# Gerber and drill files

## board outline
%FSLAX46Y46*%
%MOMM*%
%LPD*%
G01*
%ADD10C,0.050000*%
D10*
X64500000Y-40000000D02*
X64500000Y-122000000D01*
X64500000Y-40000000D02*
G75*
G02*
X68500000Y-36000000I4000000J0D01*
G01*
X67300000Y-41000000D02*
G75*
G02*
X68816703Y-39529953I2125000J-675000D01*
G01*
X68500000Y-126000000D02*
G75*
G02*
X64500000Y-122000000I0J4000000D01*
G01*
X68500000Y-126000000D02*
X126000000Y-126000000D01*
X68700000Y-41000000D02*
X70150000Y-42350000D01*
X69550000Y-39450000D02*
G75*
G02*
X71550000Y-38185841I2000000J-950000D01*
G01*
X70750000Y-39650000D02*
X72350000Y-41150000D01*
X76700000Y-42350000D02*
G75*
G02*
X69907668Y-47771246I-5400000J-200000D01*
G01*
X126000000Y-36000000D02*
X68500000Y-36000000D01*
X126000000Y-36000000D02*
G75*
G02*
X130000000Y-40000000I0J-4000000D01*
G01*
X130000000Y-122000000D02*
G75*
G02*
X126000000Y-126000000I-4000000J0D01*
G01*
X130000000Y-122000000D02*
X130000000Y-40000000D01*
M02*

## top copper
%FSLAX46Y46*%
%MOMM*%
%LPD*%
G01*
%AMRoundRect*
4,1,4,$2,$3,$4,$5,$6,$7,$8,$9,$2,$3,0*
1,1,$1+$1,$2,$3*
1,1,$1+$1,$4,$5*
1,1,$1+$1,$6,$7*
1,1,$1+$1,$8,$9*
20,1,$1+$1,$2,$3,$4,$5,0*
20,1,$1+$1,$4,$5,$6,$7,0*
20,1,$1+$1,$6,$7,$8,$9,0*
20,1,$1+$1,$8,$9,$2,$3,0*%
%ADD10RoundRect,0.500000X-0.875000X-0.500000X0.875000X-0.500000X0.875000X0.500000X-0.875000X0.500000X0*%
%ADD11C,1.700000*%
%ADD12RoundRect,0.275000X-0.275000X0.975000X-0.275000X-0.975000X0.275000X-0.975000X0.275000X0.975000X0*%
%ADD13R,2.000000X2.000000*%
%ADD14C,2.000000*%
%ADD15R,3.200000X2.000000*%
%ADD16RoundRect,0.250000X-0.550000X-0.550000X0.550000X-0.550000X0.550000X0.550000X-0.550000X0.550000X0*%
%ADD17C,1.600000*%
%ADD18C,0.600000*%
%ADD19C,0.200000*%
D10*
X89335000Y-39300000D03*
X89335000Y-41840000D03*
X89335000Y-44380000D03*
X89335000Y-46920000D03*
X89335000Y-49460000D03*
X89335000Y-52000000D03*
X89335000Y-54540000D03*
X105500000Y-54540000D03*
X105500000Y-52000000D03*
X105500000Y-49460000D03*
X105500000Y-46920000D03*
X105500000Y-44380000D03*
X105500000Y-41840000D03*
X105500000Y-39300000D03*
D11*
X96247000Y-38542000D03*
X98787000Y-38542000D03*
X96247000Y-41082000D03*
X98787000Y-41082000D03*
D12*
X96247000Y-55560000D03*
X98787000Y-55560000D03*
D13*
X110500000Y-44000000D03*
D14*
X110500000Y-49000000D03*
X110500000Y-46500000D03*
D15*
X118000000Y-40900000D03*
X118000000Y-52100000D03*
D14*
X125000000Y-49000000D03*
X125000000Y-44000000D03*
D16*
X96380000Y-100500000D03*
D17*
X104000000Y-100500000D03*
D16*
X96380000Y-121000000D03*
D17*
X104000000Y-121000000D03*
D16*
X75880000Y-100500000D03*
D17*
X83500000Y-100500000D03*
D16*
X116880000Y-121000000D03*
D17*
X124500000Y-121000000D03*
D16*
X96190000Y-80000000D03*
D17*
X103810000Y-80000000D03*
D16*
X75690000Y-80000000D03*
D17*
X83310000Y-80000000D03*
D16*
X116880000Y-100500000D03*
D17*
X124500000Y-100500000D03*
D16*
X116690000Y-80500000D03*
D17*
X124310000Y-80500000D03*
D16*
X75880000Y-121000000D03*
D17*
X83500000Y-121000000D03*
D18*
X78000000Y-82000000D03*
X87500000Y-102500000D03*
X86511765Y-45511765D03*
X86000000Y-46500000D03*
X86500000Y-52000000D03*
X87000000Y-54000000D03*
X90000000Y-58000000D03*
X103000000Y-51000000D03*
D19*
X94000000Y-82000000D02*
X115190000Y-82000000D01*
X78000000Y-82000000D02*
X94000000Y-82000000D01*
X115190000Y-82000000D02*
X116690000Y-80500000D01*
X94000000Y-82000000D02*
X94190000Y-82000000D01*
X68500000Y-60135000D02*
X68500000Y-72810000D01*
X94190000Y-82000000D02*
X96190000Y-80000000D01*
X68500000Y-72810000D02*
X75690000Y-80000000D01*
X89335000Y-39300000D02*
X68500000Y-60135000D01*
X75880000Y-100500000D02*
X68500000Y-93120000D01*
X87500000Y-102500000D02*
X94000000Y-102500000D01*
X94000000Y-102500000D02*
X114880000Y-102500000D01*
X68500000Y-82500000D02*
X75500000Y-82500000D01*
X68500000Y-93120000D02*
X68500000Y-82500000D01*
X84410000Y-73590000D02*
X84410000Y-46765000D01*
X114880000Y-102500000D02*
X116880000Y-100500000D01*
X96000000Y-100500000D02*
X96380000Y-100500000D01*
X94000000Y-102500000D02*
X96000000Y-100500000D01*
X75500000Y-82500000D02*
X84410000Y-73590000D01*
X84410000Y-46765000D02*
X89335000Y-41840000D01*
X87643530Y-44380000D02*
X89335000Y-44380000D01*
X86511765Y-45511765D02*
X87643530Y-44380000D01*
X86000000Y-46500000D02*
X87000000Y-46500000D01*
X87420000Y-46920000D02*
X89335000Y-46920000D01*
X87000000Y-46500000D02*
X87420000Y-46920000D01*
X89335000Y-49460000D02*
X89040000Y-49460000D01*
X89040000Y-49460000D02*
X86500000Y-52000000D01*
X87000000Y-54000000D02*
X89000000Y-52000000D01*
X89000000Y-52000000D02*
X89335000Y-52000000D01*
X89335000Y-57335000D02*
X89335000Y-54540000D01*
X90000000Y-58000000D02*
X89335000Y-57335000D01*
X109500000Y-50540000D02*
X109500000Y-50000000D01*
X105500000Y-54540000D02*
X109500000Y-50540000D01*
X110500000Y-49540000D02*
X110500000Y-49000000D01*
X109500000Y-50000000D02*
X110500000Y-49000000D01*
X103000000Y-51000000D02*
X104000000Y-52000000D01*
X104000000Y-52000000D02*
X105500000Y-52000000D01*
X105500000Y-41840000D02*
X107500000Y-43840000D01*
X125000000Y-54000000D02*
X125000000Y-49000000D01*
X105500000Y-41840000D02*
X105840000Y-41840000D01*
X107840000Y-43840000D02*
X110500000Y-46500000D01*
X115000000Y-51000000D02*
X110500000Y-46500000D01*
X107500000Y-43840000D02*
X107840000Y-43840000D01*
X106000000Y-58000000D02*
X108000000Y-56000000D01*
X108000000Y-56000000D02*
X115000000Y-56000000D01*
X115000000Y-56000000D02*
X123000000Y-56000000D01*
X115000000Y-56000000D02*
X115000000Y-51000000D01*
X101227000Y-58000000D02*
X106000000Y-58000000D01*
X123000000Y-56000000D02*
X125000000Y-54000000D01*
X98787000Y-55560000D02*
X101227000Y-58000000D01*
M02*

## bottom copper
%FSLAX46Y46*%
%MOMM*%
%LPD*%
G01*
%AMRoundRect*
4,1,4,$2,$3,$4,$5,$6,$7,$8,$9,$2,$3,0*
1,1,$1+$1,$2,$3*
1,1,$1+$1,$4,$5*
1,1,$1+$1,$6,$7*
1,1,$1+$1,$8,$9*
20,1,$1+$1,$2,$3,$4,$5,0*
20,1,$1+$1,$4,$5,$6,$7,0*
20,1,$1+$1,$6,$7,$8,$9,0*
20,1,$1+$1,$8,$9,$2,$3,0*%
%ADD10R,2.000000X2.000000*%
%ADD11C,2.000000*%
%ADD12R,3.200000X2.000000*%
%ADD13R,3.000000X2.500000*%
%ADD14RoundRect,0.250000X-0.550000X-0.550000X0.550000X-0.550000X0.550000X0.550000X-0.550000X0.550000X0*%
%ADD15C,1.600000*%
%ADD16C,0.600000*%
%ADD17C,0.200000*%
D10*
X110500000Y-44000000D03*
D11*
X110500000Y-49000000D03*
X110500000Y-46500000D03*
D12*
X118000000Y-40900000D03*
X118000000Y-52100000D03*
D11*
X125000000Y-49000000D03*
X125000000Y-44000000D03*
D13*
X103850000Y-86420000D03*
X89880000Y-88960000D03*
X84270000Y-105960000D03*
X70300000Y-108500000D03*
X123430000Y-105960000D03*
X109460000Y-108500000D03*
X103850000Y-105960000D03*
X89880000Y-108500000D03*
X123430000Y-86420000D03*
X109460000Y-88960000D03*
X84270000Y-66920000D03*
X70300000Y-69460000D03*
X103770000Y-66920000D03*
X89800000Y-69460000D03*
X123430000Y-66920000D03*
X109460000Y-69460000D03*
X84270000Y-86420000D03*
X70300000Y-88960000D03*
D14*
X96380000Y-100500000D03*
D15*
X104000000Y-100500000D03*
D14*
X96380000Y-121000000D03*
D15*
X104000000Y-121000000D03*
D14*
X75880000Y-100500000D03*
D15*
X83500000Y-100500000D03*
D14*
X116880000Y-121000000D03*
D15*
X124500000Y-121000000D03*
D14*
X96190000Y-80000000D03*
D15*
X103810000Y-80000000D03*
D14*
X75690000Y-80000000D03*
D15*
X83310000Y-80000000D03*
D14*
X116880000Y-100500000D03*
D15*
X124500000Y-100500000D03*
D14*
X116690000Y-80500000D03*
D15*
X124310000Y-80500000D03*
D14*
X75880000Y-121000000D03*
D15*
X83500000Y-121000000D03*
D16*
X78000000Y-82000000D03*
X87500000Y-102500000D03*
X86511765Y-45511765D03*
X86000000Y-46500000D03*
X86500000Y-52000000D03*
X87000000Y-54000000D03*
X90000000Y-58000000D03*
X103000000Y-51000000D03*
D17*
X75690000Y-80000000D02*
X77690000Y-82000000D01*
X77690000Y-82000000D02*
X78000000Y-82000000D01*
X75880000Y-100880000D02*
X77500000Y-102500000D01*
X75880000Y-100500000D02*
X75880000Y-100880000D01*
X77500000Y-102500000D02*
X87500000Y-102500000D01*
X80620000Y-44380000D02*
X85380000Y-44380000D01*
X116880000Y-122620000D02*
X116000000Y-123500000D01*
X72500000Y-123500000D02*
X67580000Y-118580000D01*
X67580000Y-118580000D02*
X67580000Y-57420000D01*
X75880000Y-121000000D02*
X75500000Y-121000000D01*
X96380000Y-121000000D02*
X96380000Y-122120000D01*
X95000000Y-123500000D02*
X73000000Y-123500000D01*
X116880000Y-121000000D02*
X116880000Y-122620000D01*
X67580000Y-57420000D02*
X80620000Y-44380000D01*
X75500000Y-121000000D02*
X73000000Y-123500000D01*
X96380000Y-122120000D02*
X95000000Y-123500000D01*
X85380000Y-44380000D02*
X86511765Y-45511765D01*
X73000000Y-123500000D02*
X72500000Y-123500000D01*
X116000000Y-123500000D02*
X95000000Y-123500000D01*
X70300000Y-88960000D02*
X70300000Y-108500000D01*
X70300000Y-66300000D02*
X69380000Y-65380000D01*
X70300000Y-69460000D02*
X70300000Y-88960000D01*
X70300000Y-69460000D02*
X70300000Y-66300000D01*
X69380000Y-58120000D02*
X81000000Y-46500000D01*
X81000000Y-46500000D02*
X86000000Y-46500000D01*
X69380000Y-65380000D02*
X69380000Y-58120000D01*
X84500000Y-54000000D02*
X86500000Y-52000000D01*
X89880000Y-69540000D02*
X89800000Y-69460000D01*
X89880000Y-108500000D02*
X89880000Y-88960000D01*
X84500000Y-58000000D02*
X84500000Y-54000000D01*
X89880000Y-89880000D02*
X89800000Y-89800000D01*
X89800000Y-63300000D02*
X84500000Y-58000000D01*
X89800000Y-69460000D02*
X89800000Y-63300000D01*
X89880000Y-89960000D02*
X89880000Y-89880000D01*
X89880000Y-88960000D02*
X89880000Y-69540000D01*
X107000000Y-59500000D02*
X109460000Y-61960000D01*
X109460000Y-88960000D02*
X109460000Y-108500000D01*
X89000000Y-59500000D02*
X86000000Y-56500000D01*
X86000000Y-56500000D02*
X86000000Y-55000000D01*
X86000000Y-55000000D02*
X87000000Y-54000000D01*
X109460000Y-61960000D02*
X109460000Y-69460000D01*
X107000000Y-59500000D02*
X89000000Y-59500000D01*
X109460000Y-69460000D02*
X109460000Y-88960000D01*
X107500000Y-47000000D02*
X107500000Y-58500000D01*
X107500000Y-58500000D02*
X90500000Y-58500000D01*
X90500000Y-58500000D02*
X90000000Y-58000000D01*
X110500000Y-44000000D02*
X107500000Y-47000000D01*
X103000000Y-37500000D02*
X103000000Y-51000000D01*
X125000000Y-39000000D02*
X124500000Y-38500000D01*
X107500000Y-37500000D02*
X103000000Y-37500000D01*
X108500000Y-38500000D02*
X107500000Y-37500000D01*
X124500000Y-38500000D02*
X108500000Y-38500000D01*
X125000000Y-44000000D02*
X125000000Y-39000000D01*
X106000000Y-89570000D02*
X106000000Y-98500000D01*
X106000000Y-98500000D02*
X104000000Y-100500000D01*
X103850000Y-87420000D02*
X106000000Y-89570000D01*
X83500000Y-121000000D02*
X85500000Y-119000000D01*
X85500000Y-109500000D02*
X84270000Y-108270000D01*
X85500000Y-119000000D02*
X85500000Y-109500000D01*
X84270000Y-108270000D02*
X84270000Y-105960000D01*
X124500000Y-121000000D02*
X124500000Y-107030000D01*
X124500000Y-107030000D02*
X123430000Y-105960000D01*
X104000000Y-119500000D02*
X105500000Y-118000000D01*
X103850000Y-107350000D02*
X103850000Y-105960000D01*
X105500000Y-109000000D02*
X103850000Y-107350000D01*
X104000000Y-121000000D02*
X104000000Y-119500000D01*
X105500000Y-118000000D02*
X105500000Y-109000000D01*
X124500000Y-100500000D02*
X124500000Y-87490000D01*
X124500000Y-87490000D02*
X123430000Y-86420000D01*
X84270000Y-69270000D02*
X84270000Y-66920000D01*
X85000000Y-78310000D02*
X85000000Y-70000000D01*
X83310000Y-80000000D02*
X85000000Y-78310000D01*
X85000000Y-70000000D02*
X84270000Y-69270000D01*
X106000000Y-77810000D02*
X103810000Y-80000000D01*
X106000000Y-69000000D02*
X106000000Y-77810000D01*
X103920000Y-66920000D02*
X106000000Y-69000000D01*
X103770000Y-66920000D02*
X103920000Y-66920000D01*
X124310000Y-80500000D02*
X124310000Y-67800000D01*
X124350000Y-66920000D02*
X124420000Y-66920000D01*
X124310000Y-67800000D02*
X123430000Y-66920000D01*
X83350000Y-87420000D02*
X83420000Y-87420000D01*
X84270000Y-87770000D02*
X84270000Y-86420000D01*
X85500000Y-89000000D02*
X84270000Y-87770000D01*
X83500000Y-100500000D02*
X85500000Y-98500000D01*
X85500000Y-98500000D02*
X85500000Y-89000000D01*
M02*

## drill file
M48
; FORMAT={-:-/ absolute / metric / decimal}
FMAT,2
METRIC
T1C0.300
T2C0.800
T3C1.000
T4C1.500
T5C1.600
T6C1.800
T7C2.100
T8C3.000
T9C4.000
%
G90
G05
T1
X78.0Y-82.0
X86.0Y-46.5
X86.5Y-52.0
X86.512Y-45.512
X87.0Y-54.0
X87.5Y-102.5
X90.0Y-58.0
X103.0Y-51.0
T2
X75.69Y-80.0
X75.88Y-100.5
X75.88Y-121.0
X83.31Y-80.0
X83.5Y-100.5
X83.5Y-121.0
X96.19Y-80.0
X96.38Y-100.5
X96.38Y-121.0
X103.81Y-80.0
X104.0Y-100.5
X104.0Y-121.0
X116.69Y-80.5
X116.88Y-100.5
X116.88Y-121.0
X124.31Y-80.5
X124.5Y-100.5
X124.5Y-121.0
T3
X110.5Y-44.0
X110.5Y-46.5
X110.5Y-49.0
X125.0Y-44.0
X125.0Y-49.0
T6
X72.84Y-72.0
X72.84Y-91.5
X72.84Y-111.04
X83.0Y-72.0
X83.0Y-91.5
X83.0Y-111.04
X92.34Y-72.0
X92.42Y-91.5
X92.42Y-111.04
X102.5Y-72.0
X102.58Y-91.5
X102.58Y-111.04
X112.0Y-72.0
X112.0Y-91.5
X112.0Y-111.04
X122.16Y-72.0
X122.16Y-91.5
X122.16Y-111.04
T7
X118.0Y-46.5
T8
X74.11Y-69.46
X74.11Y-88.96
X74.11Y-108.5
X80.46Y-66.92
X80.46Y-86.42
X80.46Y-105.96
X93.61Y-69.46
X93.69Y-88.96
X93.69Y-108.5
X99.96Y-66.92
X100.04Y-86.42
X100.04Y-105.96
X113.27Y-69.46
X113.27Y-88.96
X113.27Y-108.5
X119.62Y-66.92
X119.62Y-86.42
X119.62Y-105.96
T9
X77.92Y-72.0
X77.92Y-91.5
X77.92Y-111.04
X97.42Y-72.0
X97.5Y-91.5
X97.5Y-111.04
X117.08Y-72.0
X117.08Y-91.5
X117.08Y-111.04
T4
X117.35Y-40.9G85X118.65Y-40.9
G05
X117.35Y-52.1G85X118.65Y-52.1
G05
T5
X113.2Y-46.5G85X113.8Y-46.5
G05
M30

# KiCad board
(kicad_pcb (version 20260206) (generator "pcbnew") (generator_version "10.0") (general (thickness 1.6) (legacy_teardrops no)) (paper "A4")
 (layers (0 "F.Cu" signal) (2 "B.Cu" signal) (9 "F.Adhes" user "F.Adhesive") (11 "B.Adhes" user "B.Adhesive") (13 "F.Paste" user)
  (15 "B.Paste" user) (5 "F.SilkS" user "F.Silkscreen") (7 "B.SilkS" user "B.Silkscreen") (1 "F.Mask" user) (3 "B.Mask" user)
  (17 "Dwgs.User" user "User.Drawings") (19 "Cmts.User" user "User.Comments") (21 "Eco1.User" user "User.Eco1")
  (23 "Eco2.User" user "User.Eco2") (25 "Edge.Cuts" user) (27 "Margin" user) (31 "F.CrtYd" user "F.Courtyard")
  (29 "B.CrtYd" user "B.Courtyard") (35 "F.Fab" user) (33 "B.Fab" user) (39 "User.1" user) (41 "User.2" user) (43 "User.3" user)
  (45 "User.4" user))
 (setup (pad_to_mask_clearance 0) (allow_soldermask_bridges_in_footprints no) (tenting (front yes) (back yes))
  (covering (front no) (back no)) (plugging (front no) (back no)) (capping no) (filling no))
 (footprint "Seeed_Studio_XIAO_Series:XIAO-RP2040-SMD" (layer "F.Cu") (at 88.5 57.42)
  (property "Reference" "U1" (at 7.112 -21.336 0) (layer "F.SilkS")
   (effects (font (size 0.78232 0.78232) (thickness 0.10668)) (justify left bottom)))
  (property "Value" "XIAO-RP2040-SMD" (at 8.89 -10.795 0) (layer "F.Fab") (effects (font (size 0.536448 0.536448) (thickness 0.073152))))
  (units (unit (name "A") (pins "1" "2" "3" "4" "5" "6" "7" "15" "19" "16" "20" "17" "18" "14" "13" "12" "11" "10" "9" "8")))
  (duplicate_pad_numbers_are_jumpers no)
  (pad "1" smd roundrect (at 0.835 -18.12) (size 2.75 2) (layers "F.Cu" "F.Mask" "F.Paste") (roundrect_rratio 0.25) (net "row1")
   (solder_mask_margin 0.0508) (thermal_bridge_angle 45))
  (pad "2" smd roundrect (at 0.835 -15.58) (size 2.75 2) (layers "F.Cu" "F.Mask" "F.Paste") (roundrect_rratio 0.25) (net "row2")
   (solder_mask_margin 0.0508) (thermal_bridge_angle 45))
  (pad "3" smd roundrect (at 0.835 -13.04) (size 2.75 2) (layers "F.Cu" "F.Mask" "F.Paste") (roundrect_rratio 0.25) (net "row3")
   (solder_mask_margin 0.0508) (thermal_bridge_angle 45))
  (pad "4" smd roundrect (at 0.835 -10.5) (size 2.75 2) (layers "F.Cu" "F.Mask" "F.Paste") (roundrect_rratio 0.25) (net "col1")
   (solder_mask_margin 0.0508) (thermal_bridge_angle 45))
  (pad "5" smd roundrect (at 0.835 -7.96) (size 2.75 2) (layers "F.Cu" "F.Mask" "F.Paste") (roundrect_rratio 0.25) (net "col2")
   (solder_mask_margin 0.0508) (thermal_bridge_angle 45))
  (pad "6" smd roundrect (at 0.835 -5.42) (size 2.75 2) (layers "F.Cu" "F.Mask" "F.Paste") (roundrect_rratio 0.25) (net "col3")
   (solder_mask_margin 0.0508) (thermal_bridge_angle 45))
  (pad "7" smd roundrect (at 0.835 -2.88) (size 2.75 2) (layers "F.Cu" "F.Mask" "F.Paste") (roundrect_rratio 0.25) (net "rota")
   (solder_mask_margin 0.0508) (thermal_bridge_angle 45))
  (pad "8" smd roundrect (at 17 -2.88) (size 2.75 2) (layers "F.Cu" "F.Mask" "F.Paste") (roundrect_rratio 0.25) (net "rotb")
   (solder_mask_margin 0.0508) (thermal_bridge_angle 45))
  (pad "9" smd roundrect (at 17 -5.42) (size 2.75 2) (layers "F.Cu" "F.Mask" "F.Paste") (roundrect_rratio 0.25) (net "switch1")
   (solder_mask_margin 0.0508) (thermal_bridge_angle 45))
  (pad "10" smd roundrect (at 17 -7.96) (size 2.75 2) (layers "F.Cu" "F.Mask" "F.Paste") (roundrect_rratio 0.25)
   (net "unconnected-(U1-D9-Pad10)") (solder_mask_margin 0.0508) (thermal_bridge_angle 45))
  (pad "11" smd roundrect (at 17 -10.5) (size 2.75 2) (layers "F.Cu" "F.Mask" "F.Paste") (roundrect_rratio 0.25)
   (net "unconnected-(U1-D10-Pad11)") (solder_mask_margin 0.0508) (thermal_bridge_angle 45))
  (pad "12" smd roundrect (at 17 -13.04) (size 2.75 2) (layers "F.Cu" "F.Mask" "F.Paste") (roundrect_rratio 0.25) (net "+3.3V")
   (solder_mask_margin 0.0508) (thermal_bridge_angle 45))
  (pad "13" smd roundrect (at 17 -15.58) (size 2.75 2) (layers "F.Cu" "F.Mask" "F.Paste") (roundrect_rratio 0.25) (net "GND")
   (solder_mask_margin 0.0508) (thermal_bridge_angle 45))
  (pad "14" smd roundrect (at 17 -18.12) (size 2.75 2) (layers "F.Cu" "F.Mask" "F.Paste") (roundrect_rratio 0.25)
   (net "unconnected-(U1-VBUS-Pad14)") (solder_mask_margin 0.0508) (thermal_bridge_angle 45))
  (pad "15" smd circle (at 7.747 -18.878) (size 1.7 1.7) (layers "F.Cu" "F.Mask" "F.Paste") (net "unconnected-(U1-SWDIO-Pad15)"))
  (pad "16" smd circle (at 10.287 -18.878) (size 1.7 1.7) (layers "F.Cu" "F.Mask" "F.Paste") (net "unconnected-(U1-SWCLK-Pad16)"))
  (pad "17" smd circle (at 7.747 -16.338) (size 1.7 1.7) (layers "F.Cu" "F.Mask" "F.Paste") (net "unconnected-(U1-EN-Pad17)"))
  (pad "18" smd circle (at 10.287 -16.338) (size 1.7 1.7) (layers "F.Cu" "F.Mask" "F.Paste") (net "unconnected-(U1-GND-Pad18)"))
  (pad "19" smd roundrect (at 7.747 -1.86 270) (size 2.5 1.1) (layers "F.Cu" "F.Mask" "F.Paste") (roundrect_rratio 0.25)
   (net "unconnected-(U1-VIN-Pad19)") (thermal_bridge_angle 45))
  (pad "20" smd roundrect (at 10.287 -1.86 270) (size 2.5 1.1) (layers "F.Cu" "F.Mask" "F.Paste") (roundrect_rratio 0.25) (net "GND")
   (thermal_bridge_angle 45)))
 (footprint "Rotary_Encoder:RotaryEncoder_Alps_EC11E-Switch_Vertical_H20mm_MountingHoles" (layer "F.Cu") (at 110.5 44)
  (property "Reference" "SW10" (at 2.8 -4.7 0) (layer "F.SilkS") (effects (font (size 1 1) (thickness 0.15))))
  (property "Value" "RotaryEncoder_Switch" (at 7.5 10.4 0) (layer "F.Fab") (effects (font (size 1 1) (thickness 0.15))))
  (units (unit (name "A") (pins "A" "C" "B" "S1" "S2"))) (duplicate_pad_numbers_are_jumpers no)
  (pad "" np_thru_hole oval (at 3 2.5) (size 2.2 1.6) (drill oval 2.2 1.6) (layers "*.Mask"))
  (pad "" np_thru_hole circle (at 7.5 2.5) (size 2.1 2.1) (drill 2.1) (layers "*.Mask"))
  (pad "A" thru_hole rect (at 0 0) (size 2 2) (drill 1) (layers "*.Cu" "*.Mask") (remove_unused_layers no) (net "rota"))
  (pad "B" thru_hole circle (at 0 5) (size 2 2) (drill 1) (layers "*.Cu" "*.Mask") (remove_unused_layers no) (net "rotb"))
  (pad "C" thru_hole circle (at 0 2.5) (size 2 2) (drill 1) (layers "*.Cu" "*.Mask") (remove_unused_layers no) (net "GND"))
  (pad "MP" thru_hole rect (at 7.5 -3.1) (size 3.2 2) (drill oval 2.8 1.5) (layers "*.Cu" "*.Mask") (remove_unused_layers no))
  (pad "MP" thru_hole rect (at 7.5 8.1) (size 3.2 2) (drill oval 2.8 1.5) (layers "*.Cu" "*.Mask") (remove_unused_layers no))
  (pad "S1" thru_hole circle (at 14.5 5) (size 2 2) (drill 1) (layers "*.Cu" "*.Mask") (remove_unused_layers no) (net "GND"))
  (pad "S2" thru_hole circle (at 14.5 0) (size 2 2) (drill 1) (layers "*.Cu" "*.Mask") (remove_unused_layers no) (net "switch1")))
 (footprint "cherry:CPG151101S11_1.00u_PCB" (layer "F.Cu") (at 100.04 86.42)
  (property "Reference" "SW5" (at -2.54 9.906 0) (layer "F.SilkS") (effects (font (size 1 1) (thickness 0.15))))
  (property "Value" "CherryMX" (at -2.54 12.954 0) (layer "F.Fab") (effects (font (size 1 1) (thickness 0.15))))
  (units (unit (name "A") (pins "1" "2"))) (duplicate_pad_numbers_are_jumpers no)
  (pad "" np_thru_hole circle (at -7.62 5.08) (size 1.8 1.8) (drill 1.8) (layers "*.Cu" "*.Mask"))
  (pad "" np_thru_hole circle (at -6.35 2.54) (size 3 3) (drill 3) (layers "*.Cu" "*.Mask"))
  (pad "" np_thru_hole circle (at -2.54 5.08) (size 4 4) (drill 4) (layers "*.Cu" "*.Mask"))
  (pad "" np_thru_hole circle (at 0 0) (size 3 3) (drill 3) (layers "*.Cu" "*.Mask"))
  (pad "" np_thru_hole circle (at 2.54 5.08) (size 1.8 1.8) (drill 1.8) (layers "*.Cu" "*.Mask"))
  (pad "1" smd rect (at 3.81 0) (size 3 2.5) (layers "B.Cu" "B.Mask" "B.Paste") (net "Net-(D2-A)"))
  (pad "2" smd rect (at -10.16 2.54) (size 3 2.5) (layers "B.Cu" "B.Mask" "B.Paste") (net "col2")))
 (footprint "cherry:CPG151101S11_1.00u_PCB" (layer "F.Cu") (at 80.46 105.96)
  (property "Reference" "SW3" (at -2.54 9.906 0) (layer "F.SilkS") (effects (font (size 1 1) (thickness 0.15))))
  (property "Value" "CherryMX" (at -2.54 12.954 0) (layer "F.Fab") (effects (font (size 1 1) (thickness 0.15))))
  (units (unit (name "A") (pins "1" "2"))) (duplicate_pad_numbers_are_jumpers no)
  (pad "" np_thru_hole circle (at -7.62 5.08) (size 1.8 1.8) (drill 1.8) (layers "*.Cu" "*.Mask"))
  (pad "" np_thru_hole circle (at -6.35 2.54) (size 3 3) (drill 3) (layers "*.Cu" "*.Mask"))
  (pad "" np_thru_hole circle (at -2.54 5.08) (size 4 4) (drill 4) (layers "*.Cu" "*.Mask"))
  (pad "" np_thru_hole circle (at 0 0) (size 3 3) (drill 3) (layers "*.Cu" "*.Mask"))
  (pad "" np_thru_hole circle (at 2.54 5.08) (size 1.8 1.8) (drill 1.8) (layers "*.Cu" "*.Mask"))
  (pad "1" smd rect (at 3.81 0) (size 3 2.5) (layers "B.Cu" "B.Mask" "B.Paste") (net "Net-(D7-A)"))
  (pad "2" smd rect (at -10.16 2.54) (size 3 2.5) (layers "B.Cu" "B.Mask" "B.Paste") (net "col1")))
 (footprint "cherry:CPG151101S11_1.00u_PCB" (layer "F.Cu") (at 119.62 105.96)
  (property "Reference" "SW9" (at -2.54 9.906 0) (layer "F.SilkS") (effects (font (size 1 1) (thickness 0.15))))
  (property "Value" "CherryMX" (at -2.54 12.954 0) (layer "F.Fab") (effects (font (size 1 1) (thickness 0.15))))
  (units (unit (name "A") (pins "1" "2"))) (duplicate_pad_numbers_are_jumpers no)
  (pad "" np_thru_hole circle (at -7.62 5.08) (size 1.8 1.8) (drill 1.8) (layers "*.Cu" "*.Mask"))
  (pad "" np_thru_hole circle (at -6.35 2.54) (size 3 3) (drill 3) (layers "*.Cu" "*.Mask"))
  (pad "" np_thru_hole circle (at -2.54 5.08) (size 4 4) (drill 4) (layers "*.Cu" "*.Mask"))
  (pad "" np_thru_hole circle (at 0 0) (size 3 3) (drill 3) (layers "*.Cu" "*.Mask"))
  (pad "" np_thru_hole circle (at 2.54 5.08) (size 1.8 1.8) (drill 1.8) (layers "*.Cu" "*.Mask"))
  (pad "1" smd rect (at 3.81 0) (size 3 2.5) (layers "B.Cu" "B.Mask" "B.Paste") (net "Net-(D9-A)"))
  (pad "2" smd rect (at -10.16 2.54) (size 3 2.5) (layers "B.Cu" "B.Mask" "B.Paste") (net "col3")))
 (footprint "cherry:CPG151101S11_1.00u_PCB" (layer "F.Cu") (at 100.04 105.96)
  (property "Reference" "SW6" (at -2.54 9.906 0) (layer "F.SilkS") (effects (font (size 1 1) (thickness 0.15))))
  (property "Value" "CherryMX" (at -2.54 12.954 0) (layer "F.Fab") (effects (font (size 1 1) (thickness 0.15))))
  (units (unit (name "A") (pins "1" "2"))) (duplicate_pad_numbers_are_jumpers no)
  (pad "" np_thru_hole circle (at -7.62 5.08) (size 1.8 1.8) (drill 1.8) (layers "*.Cu" "*.Mask"))
  (pad "" np_thru_hole circle (at -6.35 2.54) (size 3 3) (drill 3) (layers "*.Cu" "*.Mask"))
  (pad "" np_thru_hole circle (at -2.54 5.08) (size 4 4) (drill 4) (layers "*.Cu" "*.Mask"))
  (pad "" np_thru_hole circle (at 0 0) (size 3 3) (drill 3) (layers "*.Cu" "*.Mask"))
  (pad "" np_thru_hole circle (at 2.54 5.08) (size 1.8 1.8) (drill 1.8) (layers "*.Cu" "*.Mask"))
  (pad "1" smd rect (at 3.81 0) (size 3 2.5) (layers "B.Cu" "B.Mask" "B.Paste") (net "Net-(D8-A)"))
  (pad "2" smd rect (at -10.16 2.54) (size 3 2.5) (layers "B.Cu" "B.Mask" "B.Paste") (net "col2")))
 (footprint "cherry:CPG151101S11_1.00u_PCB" (layer "F.Cu") (at 119.62 86.42)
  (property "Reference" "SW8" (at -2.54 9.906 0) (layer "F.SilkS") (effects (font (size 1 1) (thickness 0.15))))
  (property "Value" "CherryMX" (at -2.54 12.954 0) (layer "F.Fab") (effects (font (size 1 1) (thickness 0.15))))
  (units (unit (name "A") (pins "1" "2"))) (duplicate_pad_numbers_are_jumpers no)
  (pad "" np_thru_hole circle (at -7.62 5.08) (size 1.8 1.8) (drill 1.8) (layers "*.Cu" "*.Mask"))
  (pad "" np_thru_hole circle (at -6.35 2.54) (size 3 3) (drill 3) (layers "*.Cu" "*.Mask"))
  (pad "" np_thru_hole circle (at -2.54 5.08) (size 4 4) (drill 4) (layers "*.Cu" "*.Mask"))
  (pad "" np_thru_hole circle (at 0 0) (size 3 3) (drill 3) (layers "*.Cu" "*.Mask"))
  (pad "" np_thru_hole circle (at 2.54 5.08) (size 1.8 1.8) (drill 1.8) (layers "*.Cu" "*.Mask"))
  (pad "1" smd rect (at 3.81 0) (size 3 2.5) (layers "B.Cu" "B.Mask" "B.Paste") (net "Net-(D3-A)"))
  (pad "2" smd rect (at -10.16 2.54) (size 3 2.5) (layers "B.Cu" "B.Mask" "B.Paste") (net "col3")))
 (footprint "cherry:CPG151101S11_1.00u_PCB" (layer "F.Cu") (at 80.46 66.92)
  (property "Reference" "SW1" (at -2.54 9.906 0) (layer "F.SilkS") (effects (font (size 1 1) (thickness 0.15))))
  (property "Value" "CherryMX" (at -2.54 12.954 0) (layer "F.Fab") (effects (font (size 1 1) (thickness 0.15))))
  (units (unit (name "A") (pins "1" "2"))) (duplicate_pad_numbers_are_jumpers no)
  (pad "" np_thru_hole circle (at -7.62 5.08) (size 1.8 1.8) (drill 1.8) (layers "*.Cu" "*.Mask"))
  (pad "" np_thru_hole circle (at -6.35 2.54) (size 3 3) (drill 3) (layers "*.Cu" "*.Mask"))
  (pad "" np_thru_hole circle (at -2.54 5.08) (size 4 4) (drill 4) (layers "*.Cu" "*.Mask"))
  (pad "" np_thru_hole circle (at 0 0) (size 3 3) (drill 3) (layers "*.Cu" "*.Mask"))
  (pad "" np_thru_hole circle (at 2.54 5.08) (size 1.8 1.8) (drill 1.8) (layers "*.Cu" "*.Mask"))
  (pad "1" smd rect (at 3.81 0) (size 3 2.5) (layers "B.Cu" "B.Mask" "B.Paste") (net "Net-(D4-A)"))
  (pad "2" smd rect (at -10.16 2.54) (size 3 2.5) (layers "B.Cu" "B.Mask" "B.Paste") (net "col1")))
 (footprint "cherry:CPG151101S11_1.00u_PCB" (layer "F.Cu") (at 99.96 66.92)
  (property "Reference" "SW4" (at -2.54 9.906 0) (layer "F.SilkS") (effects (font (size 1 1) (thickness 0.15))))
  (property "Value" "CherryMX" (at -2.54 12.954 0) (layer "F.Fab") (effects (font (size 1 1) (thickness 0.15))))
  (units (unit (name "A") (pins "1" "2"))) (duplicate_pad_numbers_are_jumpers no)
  (pad "" np_thru_hole circle (at -7.62 5.08) (size 1.8 1.8) (drill 1.8) (layers "*.Cu" "*.Mask"))
  (pad "" np_thru_hole circle (at -6.35 2.54) (size 3 3) (drill 3) (layers "*.Cu" "*.Mask"))
  (pad "" np_thru_hole circle (at -2.54 5.08) (size 4 4) (drill 4) (layers "*.Cu" "*.Mask"))
  (pad "" np_thru_hole circle (at 0 0) (size 3 3) (drill 3) (layers "*.Cu" "*.Mask"))
  (pad "" np_thru_hole circle (at 2.54 5.08) (size 1.8 1.8) (drill 1.8) (layers "*.Cu" "*.Mask"))
  (pad "1" smd rect (at 3.81 0) (size 3 2.5) (layers "B.Cu" "B.Mask" "B.Paste") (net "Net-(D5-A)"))
  (pad "2" smd rect (at -10.16 2.54) (size 3 2.5) (layers "B.Cu" "B.Mask" "B.Paste") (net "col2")))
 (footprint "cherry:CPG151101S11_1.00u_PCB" (layer "F.Cu") (at 119.62 66.92)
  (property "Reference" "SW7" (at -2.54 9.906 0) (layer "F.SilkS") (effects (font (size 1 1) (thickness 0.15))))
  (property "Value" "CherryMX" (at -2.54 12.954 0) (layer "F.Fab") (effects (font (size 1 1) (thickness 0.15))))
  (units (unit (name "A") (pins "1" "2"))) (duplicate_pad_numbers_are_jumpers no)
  (pad "" np_thru_hole circle (at -7.62 5.08) (size 1.8 1.8) (drill 1.8) (layers "*.Cu" "*.Mask"))
  (pad "" np_thru_hole circle (at -6.35 2.54) (size 3 3) (drill 3) (layers "*.Cu" "*.Mask"))
  (pad "" np_thru_hole circle (at -2.54 5.08) (size 4 4) (drill 4) (layers "*.Cu" "*.Mask"))
  (pad "" np_thru_hole circle (at 0 0) (size 3 3) (drill 3) (layers "*.Cu" "*.Mask"))
  (pad "" np_thru_hole circle (at 2.54 5.08) (size 1.8 1.8) (drill 1.8) (layers "*.Cu" "*.Mask"))
  (pad "1" smd rect (at 3.81 0) (size 3 2.5) (layers "B.Cu" "B.Mask" "B.Paste") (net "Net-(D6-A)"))
  (pad "2" smd rect (at -10.16 2.54) (size 3 2.5) (layers "B.Cu" "B.Mask" "B.Paste") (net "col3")))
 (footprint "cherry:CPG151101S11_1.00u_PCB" (layer "F.Cu") (at 80.46 86.42)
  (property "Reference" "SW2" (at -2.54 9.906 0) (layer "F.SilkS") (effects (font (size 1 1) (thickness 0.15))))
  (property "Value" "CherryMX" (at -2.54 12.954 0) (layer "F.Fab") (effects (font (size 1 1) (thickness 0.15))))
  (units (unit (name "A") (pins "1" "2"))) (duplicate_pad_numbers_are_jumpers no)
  (pad "" np_thru_hole circle (at -7.62 5.08) (size 1.8 1.8) (drill 1.8) (layers "*.Cu" "*.Mask"))
  (pad "" np_thru_hole circle (at -6.35 2.54) (size 3 3) (drill 3) (layers "*.Cu" "*.Mask"))
  (pad "" np_thru_hole circle (at -2.54 5.08) (size 4 4) (drill 4) (layers "*.Cu" "*.Mask"))
  (pad "" np_thru_hole circle (at 0 0) (size 3 3) (drill 3) (layers "*.Cu" "*.Mask"))
  (pad "" np_thru_hole circle (at 2.54 5.08) (size 1.8 1.8) (drill 1.8) (layers "*.Cu" "*.Mask"))
  (pad "1" smd rect (at 3.81 0) (size 3 2.5) (layers "B.Cu" "B.Mask" "B.Paste") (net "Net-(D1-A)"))
  (pad "2" smd rect (at -10.16 2.54) (size 3 2.5) (layers "B.Cu" "B.Mask" "B.Paste") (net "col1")))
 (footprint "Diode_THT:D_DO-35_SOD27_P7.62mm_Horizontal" (layer "B.Cu") (at 96.38 100.5)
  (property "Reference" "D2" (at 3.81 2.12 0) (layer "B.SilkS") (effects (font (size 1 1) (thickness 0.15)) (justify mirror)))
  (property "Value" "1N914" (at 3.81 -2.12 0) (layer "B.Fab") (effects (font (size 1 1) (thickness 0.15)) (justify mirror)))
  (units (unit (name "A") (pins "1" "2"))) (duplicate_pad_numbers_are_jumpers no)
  (pad "1" thru_hole roundrect (at 0 0) (size 1.6 1.6) (drill 0.8) (layers "*.Cu" "*.Mask") (remove_unused_layers no)
   (roundrect_rratio 0.15625) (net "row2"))
  (pad "2" thru_hole circle (at 7.62 0) (size 1.6 1.6) (drill 0.8) (layers "*.Cu" "*.Mask") (remove_unused_layers no) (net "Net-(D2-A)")))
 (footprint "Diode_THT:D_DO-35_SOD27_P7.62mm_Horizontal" (layer "B.Cu") (at 96.38 121)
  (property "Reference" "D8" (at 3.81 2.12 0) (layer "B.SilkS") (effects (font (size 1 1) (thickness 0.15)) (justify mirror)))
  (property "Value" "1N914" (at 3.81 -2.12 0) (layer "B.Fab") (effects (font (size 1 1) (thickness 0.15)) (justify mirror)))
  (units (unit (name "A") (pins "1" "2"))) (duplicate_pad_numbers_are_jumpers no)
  (pad "1" thru_hole roundrect (at 0 0) (size 1.6 1.6) (drill 0.8) (layers "*.Cu" "*.Mask") (remove_unused_layers no)
   (roundrect_rratio 0.15625) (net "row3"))
  (pad "2" thru_hole circle (at 7.62 0) (size 1.6 1.6) (drill 0.8) (layers "*.Cu" "*.Mask") (remove_unused_layers no) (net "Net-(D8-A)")))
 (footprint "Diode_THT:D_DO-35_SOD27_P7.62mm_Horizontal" (layer "B.Cu") (at 75.88 100.5)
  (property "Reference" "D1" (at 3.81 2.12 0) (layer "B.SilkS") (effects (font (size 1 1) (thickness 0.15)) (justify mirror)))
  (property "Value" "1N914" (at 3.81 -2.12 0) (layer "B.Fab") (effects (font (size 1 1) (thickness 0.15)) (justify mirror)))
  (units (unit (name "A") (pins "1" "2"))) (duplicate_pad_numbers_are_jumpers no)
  (pad "1" thru_hole roundrect (at 0 0) (size 1.6 1.6) (drill 0.8) (layers "*.Cu" "*.Mask") (remove_unused_layers no)
   (roundrect_rratio 0.15625) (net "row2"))
  (pad "2" thru_hole circle (at 7.62 0) (size 1.6 1.6) (drill 0.8) (layers "*.Cu" "*.Mask") (remove_unused_layers no) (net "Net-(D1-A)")))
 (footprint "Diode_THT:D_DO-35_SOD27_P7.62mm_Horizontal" (layer "B.Cu") (at 116.88 121)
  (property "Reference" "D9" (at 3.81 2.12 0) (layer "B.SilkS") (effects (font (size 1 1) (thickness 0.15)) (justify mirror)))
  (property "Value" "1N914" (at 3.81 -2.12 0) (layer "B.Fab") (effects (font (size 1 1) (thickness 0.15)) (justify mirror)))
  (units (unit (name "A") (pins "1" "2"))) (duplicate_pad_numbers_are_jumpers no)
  (pad "1" thru_hole roundrect (at 0 0) (size 1.6 1.6) (drill 0.8) (layers "*.Cu" "*.Mask") (remove_unused_layers no)
   (roundrect_rratio 0.15625) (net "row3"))
  (pad "2" thru_hole circle (at 7.62 0) (size 1.6 1.6) (drill 0.8) (layers "*.Cu" "*.Mask") (remove_unused_layers no) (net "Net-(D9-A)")))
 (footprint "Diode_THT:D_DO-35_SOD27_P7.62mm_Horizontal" (layer "B.Cu") (at 96.19 80)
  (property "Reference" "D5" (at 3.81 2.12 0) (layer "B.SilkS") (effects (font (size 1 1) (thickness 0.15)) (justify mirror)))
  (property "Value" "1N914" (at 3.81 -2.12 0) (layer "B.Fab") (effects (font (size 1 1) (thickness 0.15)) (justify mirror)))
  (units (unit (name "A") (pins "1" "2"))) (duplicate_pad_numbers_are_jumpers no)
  (pad "1" thru_hole roundrect (at 0 0) (size 1.6 1.6) (drill 0.8) (layers "*.Cu" "*.Mask") (remove_unused_layers no)
   (roundrect_rratio 0.15625) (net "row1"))
  (pad "2" thru_hole circle (at 7.62 0) (size 1.6 1.6) (drill 0.8) (layers "*.Cu" "*.Mask") (remove_unused_layers no) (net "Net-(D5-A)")))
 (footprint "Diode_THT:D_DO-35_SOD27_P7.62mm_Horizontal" (layer "B.Cu") (at 75.69 80)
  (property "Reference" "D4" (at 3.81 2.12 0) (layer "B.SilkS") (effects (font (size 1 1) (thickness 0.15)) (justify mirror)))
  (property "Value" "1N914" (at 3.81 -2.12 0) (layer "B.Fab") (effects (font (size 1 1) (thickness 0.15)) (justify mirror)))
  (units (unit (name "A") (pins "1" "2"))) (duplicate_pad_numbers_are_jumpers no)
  (pad "1" thru_hole roundrect (at 0 0) (size 1.6 1.6) (drill 0.8) (layers "*.Cu" "*.Mask") (remove_unused_layers no)
   (roundrect_rratio 0.15625) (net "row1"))
  (pad "2" thru_hole circle (at 7.62 0) (size 1.6 1.6) (drill 0.8) (layers "*.Cu" "*.Mask") (remove_unused_layers no) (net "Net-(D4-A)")))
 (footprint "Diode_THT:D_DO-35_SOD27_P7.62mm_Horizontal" (layer "B.Cu") (at 116.88 100.5)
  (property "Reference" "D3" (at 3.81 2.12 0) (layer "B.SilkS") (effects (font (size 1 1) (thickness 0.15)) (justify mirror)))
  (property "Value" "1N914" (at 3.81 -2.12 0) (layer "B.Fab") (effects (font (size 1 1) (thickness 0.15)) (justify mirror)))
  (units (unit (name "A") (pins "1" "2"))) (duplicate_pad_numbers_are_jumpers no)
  (pad "1" thru_hole roundrect (at 0 0) (size 1.6 1.6) (drill 0.8) (layers "*.Cu" "*.Mask") (remove_unused_layers no)
   (roundrect_rratio 0.15625) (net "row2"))
  (pad "2" thru_hole circle (at 7.62 0) (size 1.6 1.6) (drill 0.8) (layers "*.Cu" "*.Mask") (remove_unused_layers no) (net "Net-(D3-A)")))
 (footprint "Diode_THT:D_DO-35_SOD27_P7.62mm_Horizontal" (layer "B.Cu") (at 116.69 80.5)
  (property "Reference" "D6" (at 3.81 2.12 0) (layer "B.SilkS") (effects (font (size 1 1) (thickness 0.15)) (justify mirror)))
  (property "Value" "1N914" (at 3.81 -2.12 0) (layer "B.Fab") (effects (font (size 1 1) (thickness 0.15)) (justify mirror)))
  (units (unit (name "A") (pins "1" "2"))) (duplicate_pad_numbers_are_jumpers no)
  (pad "1" thru_hole roundrect (at 0 0) (size 1.6 1.6) (drill 0.8) (layers "*.Cu" "*.Mask") (remove_unused_layers no)
   (roundrect_rratio 0.15625) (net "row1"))
  (pad "2" thru_hole circle (at 7.62 0) (size 1.6 1.6) (drill 0.8) (layers "*.Cu" "*.Mask") (remove_unused_layers no) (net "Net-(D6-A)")))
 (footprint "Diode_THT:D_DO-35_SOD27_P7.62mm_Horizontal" (layer "B.Cu") (at 75.88 121)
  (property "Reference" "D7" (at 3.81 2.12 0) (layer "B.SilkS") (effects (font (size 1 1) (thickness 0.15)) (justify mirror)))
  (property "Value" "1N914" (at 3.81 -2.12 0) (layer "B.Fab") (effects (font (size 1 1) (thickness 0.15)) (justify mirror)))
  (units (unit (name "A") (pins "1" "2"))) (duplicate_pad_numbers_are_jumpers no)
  (pad "1" thru_hole roundrect (at 0 0) (size 1.6 1.6) (drill 0.8) (layers "*.Cu" "*.Mask") (remove_unused_layers no)
   (roundrect_rratio 0.15625) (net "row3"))
  (pad "2" thru_hole circle (at 7.62 0) (size 1.6 1.6) (drill 0.8) (layers "*.Cu" "*.Mask") (remove_unused_layers no) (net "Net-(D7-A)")))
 (gr_line (start 64.5 40) (end 64.5 122) (stroke (width 0.05) (type default)) (layer "Edge.Cuts"))
 (gr_arc (start 64.5 40) (mid 65.671573 37.171573) (end 68.5 36) (stroke (width 0.05) (type default)) (layer "Edge.Cuts"))
 (gr_arc (start 67.3 41) (mid 67.873231 40.073981) (end 68.816703 39.529953) (stroke (width 0.05) (type default)) (layer "Edge.Cuts"))
 (gr_arc (start 68.5 126) (mid 65.671573 124.828427) (end 64.5 122) (stroke (width 0.05) (type default)) (layer "Edge.Cuts"))
 (gr_line (start 68.5 126) (end 126 126) (stroke (width 0.05) (type default)) (layer "Edge.Cuts"))
 (gr_line (start 68.7 41) (end 70.15 42.35) (stroke (width 0.05) (type default)) (layer "Edge.Cuts"))
 (gr_arc (start 69.55 39.45) (mid 70.366985 38.528376) (end 71.55 38.185841) (stroke (width 0.05) (type default)) (layer "Edge.Cuts"))
 (gr_line (start 70.75 39.65) (end 72.35 41.15) (stroke (width 0.05) (type default)) (layer "Edge.Cuts"))
 (gr_arc (start 76.7 42.35) (mid 74.670879 46.773408) (end 69.907668 47.771246) (stroke (width 0.05) (type default)) (layer "Edge.Cuts"))
 (gr_line (start 126 36) (end 68.5 36) (stroke (width 0.05) (type default)) (layer "Edge.Cuts"))
 (gr_arc (start 126 36) (mid 128.828427 37.171573) (end 130 40) (stroke (width 0.05) (type default)) (layer "Edge.Cuts"))
 (gr_arc (start 130 122) (mid 128.828427 124.828427) (end 126 126) (stroke (width 0.05) (type default)) (layer "Edge.Cuts"))
 (gr_line (start 130 122) (end 130 40) (stroke (width 0.05) (type default)) (layer "Edge.Cuts"))
 (segment (start 94 82) (end 115.19 82) (width 0.2) (layer "F.Cu") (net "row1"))
 (segment (start 78 82) (end 94 82) (width 0.2) (layer "F.Cu") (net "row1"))
 (segment (start 115.19 82) (end 116.69 80.5) (width 0.2) (layer "F.Cu") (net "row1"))
 (segment (start 94 82) (end 94.19 82) (width 0.2) (layer "F.Cu") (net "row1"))
 (segment (start 68.5 60.135) (end 68.5 72.81) (width 0.2) (layer "F.Cu") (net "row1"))
 (segment (start 94.19 82) (end 96.19 80) (width 0.2) (layer "F.Cu") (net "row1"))
 (segment (start 68.5 72.81) (end 75.69 80) (width 0.2) (layer "F.Cu") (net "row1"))
 (segment (start 89.335 39.3) (end 68.5 60.135) (width 0.2) (layer "F.Cu") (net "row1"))
 (via (at 78 82) (size 0.6) (drill 0.3) (layers "F.Cu" "B.Cu") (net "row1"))
 (segment (start 75.69 80) (end 77.69 82) (width 0.2) (layer "B.Cu") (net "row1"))
 (segment (start 77.69 82) (end 78 82) (width 0.2) (layer "B.Cu") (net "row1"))
 (segment (start 75.88 100.5) (end 68.5 93.12) (width 0.2) (layer "F.Cu") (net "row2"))
 (segment (start 87.5 102.5) (end 94 102.5) (width 0.2) (layer "F.Cu") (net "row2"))
 (segment (start 94 102.5) (end 114.88 102.5) (width 0.2) (layer "F.Cu") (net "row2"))
 (segment (start 68.5 82.5) (end 75.5 82.5) (width 0.2) (layer "F.Cu") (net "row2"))
 (segment (start 68.5 93.12) (end 68.5 82.5) (width 0.2) (layer "F.Cu") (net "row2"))
 (segment (start 84.41 73.59) (end 84.41 46.765) (width 0.2) (layer "F.Cu") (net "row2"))
 (segment (start 114.88 102.5) (end 116.88 100.5) (width 0.2) (layer "F.Cu") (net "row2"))
 (segment (start 96 100.5) (end 96.38 100.5) (width 0.2) (layer "F.Cu") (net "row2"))
 (segment (start 94 102.5) (end 96 100.5) (width 0.2) (layer "F.Cu") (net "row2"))
 (segment (start 75.5 82.5) (end 84.41 73.59) (width 0.2) (layer "F.Cu") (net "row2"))
 (segment (start 84.41 46.765) (end 89.335 41.84) (width 0.2) (layer "F.Cu") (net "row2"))
 (via (at 87.5 102.5) (size 0.6) (drill 0.3) (layers "F.Cu" "B.Cu") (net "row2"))
 (segment (start 75.88 100.88) (end 77.5 102.5) (width 0.2) (layer "B.Cu") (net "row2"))
 (segment (start 75.88 100.5) (end 75.88 100.88) (width 0.2) (layer "B.Cu") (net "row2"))
 (segment (start 77.5 102.5) (end 87.5 102.5) (width 0.2) (layer "B.Cu") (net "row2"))
 (segment (start 87.64353 44.38) (end 89.335 44.38) (width 0.2) (layer "F.Cu") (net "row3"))
 (segment (start 86.511765 45.511765) (end 87.64353 44.38) (width 0.2) (layer "F.Cu") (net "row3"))
 (via (at 86.511765 45.511765) (size 0.6) (drill 0.3) (layers "F.Cu" "B.Cu") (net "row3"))
 (segment (start 80.62 44.38) (end 85.38 44.38) (width 0.2) (layer "B.Cu") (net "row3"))
 (segment (start 116.88 122.62) (end 116 123.5) (width 0.2) (layer "B.Cu") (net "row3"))
 (segment (start 72.5 123.5) (end 67.58 118.58) (width 0.2) (layer "B.Cu") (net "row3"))
 (segment (start 67.58 118.58) (end 67.58 57.42) (width 0.2) (layer "B.Cu") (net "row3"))
 (segment (start 75.88 121) (end 75.5 121) (width 0.2) (layer "B.Cu") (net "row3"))
 (segment (start 96.38 121) (end 96.38 122.12) (width 0.2) (layer "B.Cu") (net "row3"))
 (segment (start 95 123.5) (end 73 123.5) (width 0.2) (layer "B.Cu") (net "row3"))
 (segment (start 116.88 121) (end 116.88 122.62) (width 0.2) (layer "B.Cu") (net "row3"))
 (segment (start 67.58 57.42) (end 80.62 44.38) (width 0.2) (layer "B.Cu") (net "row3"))
 (segment (start 75.5 121) (end 73 123.5) (width 0.2) (layer "B.Cu") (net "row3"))
 (segment (start 96.38 122.12) (end 95 123.5) (width 0.2) (layer "B.Cu") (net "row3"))
 (segment (start 85.38 44.38) (end 86.511765 45.511765) (width 0.2) (layer "B.Cu") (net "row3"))
 (segment (start 73 123.5) (end 72.5 123.5) (width 0.2) (layer "B.Cu") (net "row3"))
 (segment (start 116 123.5) (end 95 123.5) (width 0.2) (layer "B.Cu") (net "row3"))
 (segment (start 86 46.5) (end 87 46.5) (width 0.2) (layer "F.Cu") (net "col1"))
 (segment (start 87.42 46.92) (end 89.335 46.92) (width 0.2) (layer "F.Cu") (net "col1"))
 (segment (start 87 46.5) (end 87.42 46.92) (width 0.2) (layer "F.Cu") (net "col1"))
 (via (at 86 46.5) (size 0.6) (drill 0.3) (layers "F.Cu" "B.Cu") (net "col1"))
 (segment (start 70.3 88.96) (end 70.3 108.5) (width 0.2) (layer "B.Cu") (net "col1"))
 (segment (start 70.3 66.3) (end 69.38 65.38) (width 0.2) (layer "B.Cu") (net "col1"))
 (segment (start 70.3 69.46) (end 70.3 88.96) (width 0.2) (layer "B.Cu") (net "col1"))
 (segment (start 70.3 69.46) (end 70.3 66.3) (width 0.2) (layer "B.Cu") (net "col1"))
 (segment (start 69.38 58.12) (end 81 46.5) (width 0.2) (layer "B.Cu") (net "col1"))
 (segment (start 81 46.5) (end 86 46.5) (width 0.2) (layer "B.Cu") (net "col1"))
 (segment (start 69.38 65.38) (end 69.38 58.12) (width 0.2) (layer "B.Cu") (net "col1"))
 (segment (start 89.335 49.46) (end 89.04 49.46) (width 0.2) (layer "F.Cu") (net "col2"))
 (segment (start 89.04 49.46) (end 86.5 52) (width 0.2) (layer "F.Cu") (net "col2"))
 (via (at 86.5 52) (size 0.6) (drill 0.3) (layers "F.Cu" "B.Cu") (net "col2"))
 (segment (start 84.5 54) (end 86.5 52) (width 0.2) (layer "B.Cu") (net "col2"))
 (segment (start 89.88 69.54) (end 89.8 69.46) (width 0.2) (layer "B.Cu") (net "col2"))
 (segment (start 89.88 108.5) (end 89.88 88.96) (width 0.2) (layer "B.Cu") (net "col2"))
 (segment (start 84.5 58) (end 84.5 54) (width 0.2) (layer "B.Cu") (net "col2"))
 (segment (start 89.88 89.88) (end 89.8 89.8) (width 0.2) (layer "B.Cu") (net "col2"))
 (segment (start 89.8 63.3) (end 84.5 58) (width 0.2) (layer "B.Cu") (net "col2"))
 (segment (start 89.8 69.46) (end 89.8 63.3) (width 0.2) (layer "B.Cu") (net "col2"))
 (segment (start 89.88 89.96) (end 89.88 89.88) (width 0.2) (layer "B.Cu") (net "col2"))
 (segment (start 89.88 88.96) (end 89.88 69.54) (width 0.2) (layer "B.Cu") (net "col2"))
 (segment (start 87 54) (end 89 52) (width 0.2) (layer "F.Cu") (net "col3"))
 (segment (start 89 52) (end 89.335 52) (width 0.2) (layer "F.Cu") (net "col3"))
 (via (at 87 54) (size 0.6) (drill 0.3) (layers "F.Cu" "B.Cu") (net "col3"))
 (segment (start 107 59.5) (end 109.46 61.96) (width 0.2) (layer "B.Cu") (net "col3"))
 (segment (start 109.46 88.96) (end 109.46 108.5) (width 0.2) (layer "B.Cu") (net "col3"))
 (segment (start 89 59.5) (end 86 56.5) (width 0.2) (layer "B.Cu") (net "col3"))
 (segment (start 86 56.5) (end 86 55) (width 0.2) (layer "B.Cu") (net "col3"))
 (segment (start 86 55) (end 87 54) (width 0.2) (layer "B.Cu") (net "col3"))
 (segment (start 109.46 61.96) (end 109.46 69.46) (width 0.2) (layer "B.Cu") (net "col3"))
 (segment (start 107 59.5) (end 89 59.5) (width 0.2) (layer "B.Cu") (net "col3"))
 (segment (start 109.46 69.46) (end 109.46 88.96) (width 0.2) (layer "B.Cu") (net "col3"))
 (segment (start 89.335 57.335) (end 89.335 54.54) (width 0.2) (layer "F.Cu") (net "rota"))
 (segment (start 90 58) (end 89.335 57.335) (width 0.2) (layer "F.Cu") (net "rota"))
 (via (at 90 58) (size 0.6) (drill 0.3) (layers "F.Cu" "B.Cu") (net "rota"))
 (segment (start 107.5 47) (end 107.5 58.5) (width 0.2) (layer "B.Cu") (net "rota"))
 (segment (start 107.5 58.5) (end 90.5 58.5) (width 0.2) (layer "B.Cu") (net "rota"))
 (segment (start 90.5 58.5) (end 90 58) (width 0.2) (layer "B.Cu") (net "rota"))
 (segment (start 110.5 44) (end 107.5 47) (width 0.2) (layer "B.Cu") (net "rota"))
 (segment (start 109.5 50.54) (end 109.5 50) (width 0.2) (layer "F.Cu") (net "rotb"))
 (segment (start 105.5 54.54) (end 109.5 50.54) (width 0.2) (layer "F.Cu") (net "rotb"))
 (segment (start 110.5 49.54) (end 110.5 49) (width 0.2) (layer "F.Cu") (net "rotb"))
 (segment (start 109.5 50) (end 110.5 49) (width 0.2) (layer "F.Cu") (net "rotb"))
 (segment (start 103 51) (end 104 52) (width 0.2) (layer "F.Cu") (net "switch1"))
 (segment (start 104 52) (end 105.5 52) (width 0.2) (layer "F.Cu") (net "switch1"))
 (via (at 103 51) (size 0.6) (drill 0.3) (layers "F.Cu" "B.Cu") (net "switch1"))
 (segment (start 103 37.5) (end 103 51) (width 0.2) (layer "B.Cu") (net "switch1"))
 (segment (start 125 39) (end 124.5 38.5) (width 0.2) (layer "B.Cu") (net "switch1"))
 (segment (start 107.5 37.5) (end 103 37.5) (width 0.2) (layer "B.Cu") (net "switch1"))
 (segment (start 108.5 38.5) (end 107.5 37.5) (width 0.2) (layer "B.Cu") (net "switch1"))
 (segment (start 124.5 38.5) (end 108.5 38.5) (width 0.2) (layer "B.Cu") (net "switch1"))
 (segment (start 125 44) (end 125 39) (width 0.2) (layer "B.Cu") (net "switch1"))
 (segment (start 105.5 41.84) (end 107.5 43.84) (width 0.2) (layer "F.Cu") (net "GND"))
 (segment (start 125 54) (end 125 49) (width 0.2) (layer "F.Cu") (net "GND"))
 (segment (start 105.5 41.84) (end 105.84 41.84) (width 0.2) (layer "F.Cu") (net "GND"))
 (segment (start 107.84 43.84) (end 110.5 46.5) (width 0.2) (layer "F.Cu") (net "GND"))
 (segment (start 115 51) (end 110.5 46.5) (width 0.2) (layer "F.Cu") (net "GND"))
 (segment (start 107.5 43.84) (end 107.84 43.84) (width 0.2) (layer "F.Cu") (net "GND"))
 (segment (start 106 58) (end 108 56) (width 0.2) (layer "F.Cu") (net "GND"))
 (segment (start 108 56) (end 115 56) (width 0.2) (layer "F.Cu") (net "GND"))
 (segment (start 115 56) (end 123 56) (width 0.2) (layer "F.Cu") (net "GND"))
 (segment (start 115 56) (end 115 51) (width 0.2) (layer "F.Cu") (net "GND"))
 (segment (start 101.227 58) (end 106 58) (width 0.2) (layer "F.Cu") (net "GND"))
 (segment (start 123 56) (end 125 54) (width 0.2) (layer "F.Cu") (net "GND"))
 (segment (start 98.787 55.56) (end 101.227 58) (width 0.2) (layer "F.Cu") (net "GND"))
 (segment (start 106 89.57) (end 106 98.5) (width 0.2) (layer "B.Cu") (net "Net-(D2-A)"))
 (segment (start 106 98.5) (end 104 100.5) (width 0.2) (layer "B.Cu") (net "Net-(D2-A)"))
 (segment (start 103.85 87.42) (end 106 89.57) (width 0.2) (layer "B.Cu") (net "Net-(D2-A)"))
 (segment (start 83.5 121) (end 85.5 119) (width 0.2) (layer "B.Cu") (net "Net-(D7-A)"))
 (segment (start 85.5 109.5) (end 84.27 108.27) (width 0.2) (layer "B.Cu") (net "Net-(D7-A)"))
 (segment (start 85.5 119) (end 85.5 109.5) (width 0.2) (layer "B.Cu") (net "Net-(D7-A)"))
 (segment (start 84.27 108.27) (end 84.27 105.96) (width 0.2) (layer "B.Cu") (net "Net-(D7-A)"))
 (segment (start 124.5 121) (end 124.5 107.03) (width 0.2) (layer "B.Cu") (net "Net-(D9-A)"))
 (segment (start 124.5 107.03) (end 123.43 105.96) (width 0.2) (layer "B.Cu") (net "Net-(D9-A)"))
 (segment (start 104 119.5) (end 105.5 118) (width 0.2) (layer "B.Cu") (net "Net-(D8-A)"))
 (segment (start 103.85 107.35) (end 103.85 105.96) (width 0.2) (layer "B.Cu") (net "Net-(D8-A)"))
 (segment (start 105.5 109) (end 103.85 107.35) (width 0.2) (layer "B.Cu") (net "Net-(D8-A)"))
 (segment (start 104 121) (end 104 119.5) (width 0.2) (layer "B.Cu") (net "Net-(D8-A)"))
 (segment (start 105.5 118) (end 105.5 109) (width 0.2) (layer "B.Cu") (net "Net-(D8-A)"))
 (segment (start 124.5 100.5) (end 124.5 87.49) (width 0.2) (layer "B.Cu") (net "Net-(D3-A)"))
 (segment (start 124.5 87.49) (end 123.43 86.42) (width 0.2) (layer "B.Cu") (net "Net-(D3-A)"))
 (segment (start 84.27 69.27) (end 84.27 66.92) (width 0.2) (layer "B.Cu") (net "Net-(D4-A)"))
 (segment (start 85 78.31) (end 85 70) (width 0.2) (layer "B.Cu") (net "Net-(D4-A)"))
 (segment (start 83.31 80) (end 85 78.31) (width 0.2) (layer "B.Cu") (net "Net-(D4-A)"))
 (segment (start 85 70) (end 84.27 69.27) (width 0.2) (layer "B.Cu") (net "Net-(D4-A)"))
 (segment (start 106 77.81) (end 103.81 80) (width 0.2) (layer "B.Cu") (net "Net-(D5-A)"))
 (segment (start 106 69) (end 106 77.81) (width 0.2) (layer "B.Cu") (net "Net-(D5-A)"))
 (segment (start 103.92 66.92) (end 106 69) (width 0.2) (layer "B.Cu") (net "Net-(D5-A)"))
 (segment (start 103.77 66.92) (end 103.92 66.92) (width 0.2) (layer "B.Cu") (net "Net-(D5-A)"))
 (segment (start 124.31 80.5) (end 124.31 67.8) (width 0.2) (layer "B.Cu") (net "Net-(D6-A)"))
 (segment (start 124.35 66.92) (end 124.42 66.92) (width 0.2) (layer "B.Cu") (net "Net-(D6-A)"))
 (segment (start 124.31 67.8) (end 123.43 66.92) (width 0.2) (layer "B.Cu") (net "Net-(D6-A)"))
 (segment (start 83.35 87.42) (end 83.42 87.42) (width 0.2) (layer "B.Cu") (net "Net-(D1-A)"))
 (segment (start 84.27 87.77) (end 84.27 86.42) (width 0.2) (layer "B.Cu") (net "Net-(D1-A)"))
 (segment (start 85.5 89) (end 84.27 87.77) (width 0.2) (layer "B.Cu") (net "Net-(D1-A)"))
 (segment (start 83.5 100.5) (end 85.5 98.5) (width 0.2) (layer "B.Cu") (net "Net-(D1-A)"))
 (segment (start 85.5 98.5) (end 85.5 89) (width 0.2) (layer "B.Cu") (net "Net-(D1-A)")))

